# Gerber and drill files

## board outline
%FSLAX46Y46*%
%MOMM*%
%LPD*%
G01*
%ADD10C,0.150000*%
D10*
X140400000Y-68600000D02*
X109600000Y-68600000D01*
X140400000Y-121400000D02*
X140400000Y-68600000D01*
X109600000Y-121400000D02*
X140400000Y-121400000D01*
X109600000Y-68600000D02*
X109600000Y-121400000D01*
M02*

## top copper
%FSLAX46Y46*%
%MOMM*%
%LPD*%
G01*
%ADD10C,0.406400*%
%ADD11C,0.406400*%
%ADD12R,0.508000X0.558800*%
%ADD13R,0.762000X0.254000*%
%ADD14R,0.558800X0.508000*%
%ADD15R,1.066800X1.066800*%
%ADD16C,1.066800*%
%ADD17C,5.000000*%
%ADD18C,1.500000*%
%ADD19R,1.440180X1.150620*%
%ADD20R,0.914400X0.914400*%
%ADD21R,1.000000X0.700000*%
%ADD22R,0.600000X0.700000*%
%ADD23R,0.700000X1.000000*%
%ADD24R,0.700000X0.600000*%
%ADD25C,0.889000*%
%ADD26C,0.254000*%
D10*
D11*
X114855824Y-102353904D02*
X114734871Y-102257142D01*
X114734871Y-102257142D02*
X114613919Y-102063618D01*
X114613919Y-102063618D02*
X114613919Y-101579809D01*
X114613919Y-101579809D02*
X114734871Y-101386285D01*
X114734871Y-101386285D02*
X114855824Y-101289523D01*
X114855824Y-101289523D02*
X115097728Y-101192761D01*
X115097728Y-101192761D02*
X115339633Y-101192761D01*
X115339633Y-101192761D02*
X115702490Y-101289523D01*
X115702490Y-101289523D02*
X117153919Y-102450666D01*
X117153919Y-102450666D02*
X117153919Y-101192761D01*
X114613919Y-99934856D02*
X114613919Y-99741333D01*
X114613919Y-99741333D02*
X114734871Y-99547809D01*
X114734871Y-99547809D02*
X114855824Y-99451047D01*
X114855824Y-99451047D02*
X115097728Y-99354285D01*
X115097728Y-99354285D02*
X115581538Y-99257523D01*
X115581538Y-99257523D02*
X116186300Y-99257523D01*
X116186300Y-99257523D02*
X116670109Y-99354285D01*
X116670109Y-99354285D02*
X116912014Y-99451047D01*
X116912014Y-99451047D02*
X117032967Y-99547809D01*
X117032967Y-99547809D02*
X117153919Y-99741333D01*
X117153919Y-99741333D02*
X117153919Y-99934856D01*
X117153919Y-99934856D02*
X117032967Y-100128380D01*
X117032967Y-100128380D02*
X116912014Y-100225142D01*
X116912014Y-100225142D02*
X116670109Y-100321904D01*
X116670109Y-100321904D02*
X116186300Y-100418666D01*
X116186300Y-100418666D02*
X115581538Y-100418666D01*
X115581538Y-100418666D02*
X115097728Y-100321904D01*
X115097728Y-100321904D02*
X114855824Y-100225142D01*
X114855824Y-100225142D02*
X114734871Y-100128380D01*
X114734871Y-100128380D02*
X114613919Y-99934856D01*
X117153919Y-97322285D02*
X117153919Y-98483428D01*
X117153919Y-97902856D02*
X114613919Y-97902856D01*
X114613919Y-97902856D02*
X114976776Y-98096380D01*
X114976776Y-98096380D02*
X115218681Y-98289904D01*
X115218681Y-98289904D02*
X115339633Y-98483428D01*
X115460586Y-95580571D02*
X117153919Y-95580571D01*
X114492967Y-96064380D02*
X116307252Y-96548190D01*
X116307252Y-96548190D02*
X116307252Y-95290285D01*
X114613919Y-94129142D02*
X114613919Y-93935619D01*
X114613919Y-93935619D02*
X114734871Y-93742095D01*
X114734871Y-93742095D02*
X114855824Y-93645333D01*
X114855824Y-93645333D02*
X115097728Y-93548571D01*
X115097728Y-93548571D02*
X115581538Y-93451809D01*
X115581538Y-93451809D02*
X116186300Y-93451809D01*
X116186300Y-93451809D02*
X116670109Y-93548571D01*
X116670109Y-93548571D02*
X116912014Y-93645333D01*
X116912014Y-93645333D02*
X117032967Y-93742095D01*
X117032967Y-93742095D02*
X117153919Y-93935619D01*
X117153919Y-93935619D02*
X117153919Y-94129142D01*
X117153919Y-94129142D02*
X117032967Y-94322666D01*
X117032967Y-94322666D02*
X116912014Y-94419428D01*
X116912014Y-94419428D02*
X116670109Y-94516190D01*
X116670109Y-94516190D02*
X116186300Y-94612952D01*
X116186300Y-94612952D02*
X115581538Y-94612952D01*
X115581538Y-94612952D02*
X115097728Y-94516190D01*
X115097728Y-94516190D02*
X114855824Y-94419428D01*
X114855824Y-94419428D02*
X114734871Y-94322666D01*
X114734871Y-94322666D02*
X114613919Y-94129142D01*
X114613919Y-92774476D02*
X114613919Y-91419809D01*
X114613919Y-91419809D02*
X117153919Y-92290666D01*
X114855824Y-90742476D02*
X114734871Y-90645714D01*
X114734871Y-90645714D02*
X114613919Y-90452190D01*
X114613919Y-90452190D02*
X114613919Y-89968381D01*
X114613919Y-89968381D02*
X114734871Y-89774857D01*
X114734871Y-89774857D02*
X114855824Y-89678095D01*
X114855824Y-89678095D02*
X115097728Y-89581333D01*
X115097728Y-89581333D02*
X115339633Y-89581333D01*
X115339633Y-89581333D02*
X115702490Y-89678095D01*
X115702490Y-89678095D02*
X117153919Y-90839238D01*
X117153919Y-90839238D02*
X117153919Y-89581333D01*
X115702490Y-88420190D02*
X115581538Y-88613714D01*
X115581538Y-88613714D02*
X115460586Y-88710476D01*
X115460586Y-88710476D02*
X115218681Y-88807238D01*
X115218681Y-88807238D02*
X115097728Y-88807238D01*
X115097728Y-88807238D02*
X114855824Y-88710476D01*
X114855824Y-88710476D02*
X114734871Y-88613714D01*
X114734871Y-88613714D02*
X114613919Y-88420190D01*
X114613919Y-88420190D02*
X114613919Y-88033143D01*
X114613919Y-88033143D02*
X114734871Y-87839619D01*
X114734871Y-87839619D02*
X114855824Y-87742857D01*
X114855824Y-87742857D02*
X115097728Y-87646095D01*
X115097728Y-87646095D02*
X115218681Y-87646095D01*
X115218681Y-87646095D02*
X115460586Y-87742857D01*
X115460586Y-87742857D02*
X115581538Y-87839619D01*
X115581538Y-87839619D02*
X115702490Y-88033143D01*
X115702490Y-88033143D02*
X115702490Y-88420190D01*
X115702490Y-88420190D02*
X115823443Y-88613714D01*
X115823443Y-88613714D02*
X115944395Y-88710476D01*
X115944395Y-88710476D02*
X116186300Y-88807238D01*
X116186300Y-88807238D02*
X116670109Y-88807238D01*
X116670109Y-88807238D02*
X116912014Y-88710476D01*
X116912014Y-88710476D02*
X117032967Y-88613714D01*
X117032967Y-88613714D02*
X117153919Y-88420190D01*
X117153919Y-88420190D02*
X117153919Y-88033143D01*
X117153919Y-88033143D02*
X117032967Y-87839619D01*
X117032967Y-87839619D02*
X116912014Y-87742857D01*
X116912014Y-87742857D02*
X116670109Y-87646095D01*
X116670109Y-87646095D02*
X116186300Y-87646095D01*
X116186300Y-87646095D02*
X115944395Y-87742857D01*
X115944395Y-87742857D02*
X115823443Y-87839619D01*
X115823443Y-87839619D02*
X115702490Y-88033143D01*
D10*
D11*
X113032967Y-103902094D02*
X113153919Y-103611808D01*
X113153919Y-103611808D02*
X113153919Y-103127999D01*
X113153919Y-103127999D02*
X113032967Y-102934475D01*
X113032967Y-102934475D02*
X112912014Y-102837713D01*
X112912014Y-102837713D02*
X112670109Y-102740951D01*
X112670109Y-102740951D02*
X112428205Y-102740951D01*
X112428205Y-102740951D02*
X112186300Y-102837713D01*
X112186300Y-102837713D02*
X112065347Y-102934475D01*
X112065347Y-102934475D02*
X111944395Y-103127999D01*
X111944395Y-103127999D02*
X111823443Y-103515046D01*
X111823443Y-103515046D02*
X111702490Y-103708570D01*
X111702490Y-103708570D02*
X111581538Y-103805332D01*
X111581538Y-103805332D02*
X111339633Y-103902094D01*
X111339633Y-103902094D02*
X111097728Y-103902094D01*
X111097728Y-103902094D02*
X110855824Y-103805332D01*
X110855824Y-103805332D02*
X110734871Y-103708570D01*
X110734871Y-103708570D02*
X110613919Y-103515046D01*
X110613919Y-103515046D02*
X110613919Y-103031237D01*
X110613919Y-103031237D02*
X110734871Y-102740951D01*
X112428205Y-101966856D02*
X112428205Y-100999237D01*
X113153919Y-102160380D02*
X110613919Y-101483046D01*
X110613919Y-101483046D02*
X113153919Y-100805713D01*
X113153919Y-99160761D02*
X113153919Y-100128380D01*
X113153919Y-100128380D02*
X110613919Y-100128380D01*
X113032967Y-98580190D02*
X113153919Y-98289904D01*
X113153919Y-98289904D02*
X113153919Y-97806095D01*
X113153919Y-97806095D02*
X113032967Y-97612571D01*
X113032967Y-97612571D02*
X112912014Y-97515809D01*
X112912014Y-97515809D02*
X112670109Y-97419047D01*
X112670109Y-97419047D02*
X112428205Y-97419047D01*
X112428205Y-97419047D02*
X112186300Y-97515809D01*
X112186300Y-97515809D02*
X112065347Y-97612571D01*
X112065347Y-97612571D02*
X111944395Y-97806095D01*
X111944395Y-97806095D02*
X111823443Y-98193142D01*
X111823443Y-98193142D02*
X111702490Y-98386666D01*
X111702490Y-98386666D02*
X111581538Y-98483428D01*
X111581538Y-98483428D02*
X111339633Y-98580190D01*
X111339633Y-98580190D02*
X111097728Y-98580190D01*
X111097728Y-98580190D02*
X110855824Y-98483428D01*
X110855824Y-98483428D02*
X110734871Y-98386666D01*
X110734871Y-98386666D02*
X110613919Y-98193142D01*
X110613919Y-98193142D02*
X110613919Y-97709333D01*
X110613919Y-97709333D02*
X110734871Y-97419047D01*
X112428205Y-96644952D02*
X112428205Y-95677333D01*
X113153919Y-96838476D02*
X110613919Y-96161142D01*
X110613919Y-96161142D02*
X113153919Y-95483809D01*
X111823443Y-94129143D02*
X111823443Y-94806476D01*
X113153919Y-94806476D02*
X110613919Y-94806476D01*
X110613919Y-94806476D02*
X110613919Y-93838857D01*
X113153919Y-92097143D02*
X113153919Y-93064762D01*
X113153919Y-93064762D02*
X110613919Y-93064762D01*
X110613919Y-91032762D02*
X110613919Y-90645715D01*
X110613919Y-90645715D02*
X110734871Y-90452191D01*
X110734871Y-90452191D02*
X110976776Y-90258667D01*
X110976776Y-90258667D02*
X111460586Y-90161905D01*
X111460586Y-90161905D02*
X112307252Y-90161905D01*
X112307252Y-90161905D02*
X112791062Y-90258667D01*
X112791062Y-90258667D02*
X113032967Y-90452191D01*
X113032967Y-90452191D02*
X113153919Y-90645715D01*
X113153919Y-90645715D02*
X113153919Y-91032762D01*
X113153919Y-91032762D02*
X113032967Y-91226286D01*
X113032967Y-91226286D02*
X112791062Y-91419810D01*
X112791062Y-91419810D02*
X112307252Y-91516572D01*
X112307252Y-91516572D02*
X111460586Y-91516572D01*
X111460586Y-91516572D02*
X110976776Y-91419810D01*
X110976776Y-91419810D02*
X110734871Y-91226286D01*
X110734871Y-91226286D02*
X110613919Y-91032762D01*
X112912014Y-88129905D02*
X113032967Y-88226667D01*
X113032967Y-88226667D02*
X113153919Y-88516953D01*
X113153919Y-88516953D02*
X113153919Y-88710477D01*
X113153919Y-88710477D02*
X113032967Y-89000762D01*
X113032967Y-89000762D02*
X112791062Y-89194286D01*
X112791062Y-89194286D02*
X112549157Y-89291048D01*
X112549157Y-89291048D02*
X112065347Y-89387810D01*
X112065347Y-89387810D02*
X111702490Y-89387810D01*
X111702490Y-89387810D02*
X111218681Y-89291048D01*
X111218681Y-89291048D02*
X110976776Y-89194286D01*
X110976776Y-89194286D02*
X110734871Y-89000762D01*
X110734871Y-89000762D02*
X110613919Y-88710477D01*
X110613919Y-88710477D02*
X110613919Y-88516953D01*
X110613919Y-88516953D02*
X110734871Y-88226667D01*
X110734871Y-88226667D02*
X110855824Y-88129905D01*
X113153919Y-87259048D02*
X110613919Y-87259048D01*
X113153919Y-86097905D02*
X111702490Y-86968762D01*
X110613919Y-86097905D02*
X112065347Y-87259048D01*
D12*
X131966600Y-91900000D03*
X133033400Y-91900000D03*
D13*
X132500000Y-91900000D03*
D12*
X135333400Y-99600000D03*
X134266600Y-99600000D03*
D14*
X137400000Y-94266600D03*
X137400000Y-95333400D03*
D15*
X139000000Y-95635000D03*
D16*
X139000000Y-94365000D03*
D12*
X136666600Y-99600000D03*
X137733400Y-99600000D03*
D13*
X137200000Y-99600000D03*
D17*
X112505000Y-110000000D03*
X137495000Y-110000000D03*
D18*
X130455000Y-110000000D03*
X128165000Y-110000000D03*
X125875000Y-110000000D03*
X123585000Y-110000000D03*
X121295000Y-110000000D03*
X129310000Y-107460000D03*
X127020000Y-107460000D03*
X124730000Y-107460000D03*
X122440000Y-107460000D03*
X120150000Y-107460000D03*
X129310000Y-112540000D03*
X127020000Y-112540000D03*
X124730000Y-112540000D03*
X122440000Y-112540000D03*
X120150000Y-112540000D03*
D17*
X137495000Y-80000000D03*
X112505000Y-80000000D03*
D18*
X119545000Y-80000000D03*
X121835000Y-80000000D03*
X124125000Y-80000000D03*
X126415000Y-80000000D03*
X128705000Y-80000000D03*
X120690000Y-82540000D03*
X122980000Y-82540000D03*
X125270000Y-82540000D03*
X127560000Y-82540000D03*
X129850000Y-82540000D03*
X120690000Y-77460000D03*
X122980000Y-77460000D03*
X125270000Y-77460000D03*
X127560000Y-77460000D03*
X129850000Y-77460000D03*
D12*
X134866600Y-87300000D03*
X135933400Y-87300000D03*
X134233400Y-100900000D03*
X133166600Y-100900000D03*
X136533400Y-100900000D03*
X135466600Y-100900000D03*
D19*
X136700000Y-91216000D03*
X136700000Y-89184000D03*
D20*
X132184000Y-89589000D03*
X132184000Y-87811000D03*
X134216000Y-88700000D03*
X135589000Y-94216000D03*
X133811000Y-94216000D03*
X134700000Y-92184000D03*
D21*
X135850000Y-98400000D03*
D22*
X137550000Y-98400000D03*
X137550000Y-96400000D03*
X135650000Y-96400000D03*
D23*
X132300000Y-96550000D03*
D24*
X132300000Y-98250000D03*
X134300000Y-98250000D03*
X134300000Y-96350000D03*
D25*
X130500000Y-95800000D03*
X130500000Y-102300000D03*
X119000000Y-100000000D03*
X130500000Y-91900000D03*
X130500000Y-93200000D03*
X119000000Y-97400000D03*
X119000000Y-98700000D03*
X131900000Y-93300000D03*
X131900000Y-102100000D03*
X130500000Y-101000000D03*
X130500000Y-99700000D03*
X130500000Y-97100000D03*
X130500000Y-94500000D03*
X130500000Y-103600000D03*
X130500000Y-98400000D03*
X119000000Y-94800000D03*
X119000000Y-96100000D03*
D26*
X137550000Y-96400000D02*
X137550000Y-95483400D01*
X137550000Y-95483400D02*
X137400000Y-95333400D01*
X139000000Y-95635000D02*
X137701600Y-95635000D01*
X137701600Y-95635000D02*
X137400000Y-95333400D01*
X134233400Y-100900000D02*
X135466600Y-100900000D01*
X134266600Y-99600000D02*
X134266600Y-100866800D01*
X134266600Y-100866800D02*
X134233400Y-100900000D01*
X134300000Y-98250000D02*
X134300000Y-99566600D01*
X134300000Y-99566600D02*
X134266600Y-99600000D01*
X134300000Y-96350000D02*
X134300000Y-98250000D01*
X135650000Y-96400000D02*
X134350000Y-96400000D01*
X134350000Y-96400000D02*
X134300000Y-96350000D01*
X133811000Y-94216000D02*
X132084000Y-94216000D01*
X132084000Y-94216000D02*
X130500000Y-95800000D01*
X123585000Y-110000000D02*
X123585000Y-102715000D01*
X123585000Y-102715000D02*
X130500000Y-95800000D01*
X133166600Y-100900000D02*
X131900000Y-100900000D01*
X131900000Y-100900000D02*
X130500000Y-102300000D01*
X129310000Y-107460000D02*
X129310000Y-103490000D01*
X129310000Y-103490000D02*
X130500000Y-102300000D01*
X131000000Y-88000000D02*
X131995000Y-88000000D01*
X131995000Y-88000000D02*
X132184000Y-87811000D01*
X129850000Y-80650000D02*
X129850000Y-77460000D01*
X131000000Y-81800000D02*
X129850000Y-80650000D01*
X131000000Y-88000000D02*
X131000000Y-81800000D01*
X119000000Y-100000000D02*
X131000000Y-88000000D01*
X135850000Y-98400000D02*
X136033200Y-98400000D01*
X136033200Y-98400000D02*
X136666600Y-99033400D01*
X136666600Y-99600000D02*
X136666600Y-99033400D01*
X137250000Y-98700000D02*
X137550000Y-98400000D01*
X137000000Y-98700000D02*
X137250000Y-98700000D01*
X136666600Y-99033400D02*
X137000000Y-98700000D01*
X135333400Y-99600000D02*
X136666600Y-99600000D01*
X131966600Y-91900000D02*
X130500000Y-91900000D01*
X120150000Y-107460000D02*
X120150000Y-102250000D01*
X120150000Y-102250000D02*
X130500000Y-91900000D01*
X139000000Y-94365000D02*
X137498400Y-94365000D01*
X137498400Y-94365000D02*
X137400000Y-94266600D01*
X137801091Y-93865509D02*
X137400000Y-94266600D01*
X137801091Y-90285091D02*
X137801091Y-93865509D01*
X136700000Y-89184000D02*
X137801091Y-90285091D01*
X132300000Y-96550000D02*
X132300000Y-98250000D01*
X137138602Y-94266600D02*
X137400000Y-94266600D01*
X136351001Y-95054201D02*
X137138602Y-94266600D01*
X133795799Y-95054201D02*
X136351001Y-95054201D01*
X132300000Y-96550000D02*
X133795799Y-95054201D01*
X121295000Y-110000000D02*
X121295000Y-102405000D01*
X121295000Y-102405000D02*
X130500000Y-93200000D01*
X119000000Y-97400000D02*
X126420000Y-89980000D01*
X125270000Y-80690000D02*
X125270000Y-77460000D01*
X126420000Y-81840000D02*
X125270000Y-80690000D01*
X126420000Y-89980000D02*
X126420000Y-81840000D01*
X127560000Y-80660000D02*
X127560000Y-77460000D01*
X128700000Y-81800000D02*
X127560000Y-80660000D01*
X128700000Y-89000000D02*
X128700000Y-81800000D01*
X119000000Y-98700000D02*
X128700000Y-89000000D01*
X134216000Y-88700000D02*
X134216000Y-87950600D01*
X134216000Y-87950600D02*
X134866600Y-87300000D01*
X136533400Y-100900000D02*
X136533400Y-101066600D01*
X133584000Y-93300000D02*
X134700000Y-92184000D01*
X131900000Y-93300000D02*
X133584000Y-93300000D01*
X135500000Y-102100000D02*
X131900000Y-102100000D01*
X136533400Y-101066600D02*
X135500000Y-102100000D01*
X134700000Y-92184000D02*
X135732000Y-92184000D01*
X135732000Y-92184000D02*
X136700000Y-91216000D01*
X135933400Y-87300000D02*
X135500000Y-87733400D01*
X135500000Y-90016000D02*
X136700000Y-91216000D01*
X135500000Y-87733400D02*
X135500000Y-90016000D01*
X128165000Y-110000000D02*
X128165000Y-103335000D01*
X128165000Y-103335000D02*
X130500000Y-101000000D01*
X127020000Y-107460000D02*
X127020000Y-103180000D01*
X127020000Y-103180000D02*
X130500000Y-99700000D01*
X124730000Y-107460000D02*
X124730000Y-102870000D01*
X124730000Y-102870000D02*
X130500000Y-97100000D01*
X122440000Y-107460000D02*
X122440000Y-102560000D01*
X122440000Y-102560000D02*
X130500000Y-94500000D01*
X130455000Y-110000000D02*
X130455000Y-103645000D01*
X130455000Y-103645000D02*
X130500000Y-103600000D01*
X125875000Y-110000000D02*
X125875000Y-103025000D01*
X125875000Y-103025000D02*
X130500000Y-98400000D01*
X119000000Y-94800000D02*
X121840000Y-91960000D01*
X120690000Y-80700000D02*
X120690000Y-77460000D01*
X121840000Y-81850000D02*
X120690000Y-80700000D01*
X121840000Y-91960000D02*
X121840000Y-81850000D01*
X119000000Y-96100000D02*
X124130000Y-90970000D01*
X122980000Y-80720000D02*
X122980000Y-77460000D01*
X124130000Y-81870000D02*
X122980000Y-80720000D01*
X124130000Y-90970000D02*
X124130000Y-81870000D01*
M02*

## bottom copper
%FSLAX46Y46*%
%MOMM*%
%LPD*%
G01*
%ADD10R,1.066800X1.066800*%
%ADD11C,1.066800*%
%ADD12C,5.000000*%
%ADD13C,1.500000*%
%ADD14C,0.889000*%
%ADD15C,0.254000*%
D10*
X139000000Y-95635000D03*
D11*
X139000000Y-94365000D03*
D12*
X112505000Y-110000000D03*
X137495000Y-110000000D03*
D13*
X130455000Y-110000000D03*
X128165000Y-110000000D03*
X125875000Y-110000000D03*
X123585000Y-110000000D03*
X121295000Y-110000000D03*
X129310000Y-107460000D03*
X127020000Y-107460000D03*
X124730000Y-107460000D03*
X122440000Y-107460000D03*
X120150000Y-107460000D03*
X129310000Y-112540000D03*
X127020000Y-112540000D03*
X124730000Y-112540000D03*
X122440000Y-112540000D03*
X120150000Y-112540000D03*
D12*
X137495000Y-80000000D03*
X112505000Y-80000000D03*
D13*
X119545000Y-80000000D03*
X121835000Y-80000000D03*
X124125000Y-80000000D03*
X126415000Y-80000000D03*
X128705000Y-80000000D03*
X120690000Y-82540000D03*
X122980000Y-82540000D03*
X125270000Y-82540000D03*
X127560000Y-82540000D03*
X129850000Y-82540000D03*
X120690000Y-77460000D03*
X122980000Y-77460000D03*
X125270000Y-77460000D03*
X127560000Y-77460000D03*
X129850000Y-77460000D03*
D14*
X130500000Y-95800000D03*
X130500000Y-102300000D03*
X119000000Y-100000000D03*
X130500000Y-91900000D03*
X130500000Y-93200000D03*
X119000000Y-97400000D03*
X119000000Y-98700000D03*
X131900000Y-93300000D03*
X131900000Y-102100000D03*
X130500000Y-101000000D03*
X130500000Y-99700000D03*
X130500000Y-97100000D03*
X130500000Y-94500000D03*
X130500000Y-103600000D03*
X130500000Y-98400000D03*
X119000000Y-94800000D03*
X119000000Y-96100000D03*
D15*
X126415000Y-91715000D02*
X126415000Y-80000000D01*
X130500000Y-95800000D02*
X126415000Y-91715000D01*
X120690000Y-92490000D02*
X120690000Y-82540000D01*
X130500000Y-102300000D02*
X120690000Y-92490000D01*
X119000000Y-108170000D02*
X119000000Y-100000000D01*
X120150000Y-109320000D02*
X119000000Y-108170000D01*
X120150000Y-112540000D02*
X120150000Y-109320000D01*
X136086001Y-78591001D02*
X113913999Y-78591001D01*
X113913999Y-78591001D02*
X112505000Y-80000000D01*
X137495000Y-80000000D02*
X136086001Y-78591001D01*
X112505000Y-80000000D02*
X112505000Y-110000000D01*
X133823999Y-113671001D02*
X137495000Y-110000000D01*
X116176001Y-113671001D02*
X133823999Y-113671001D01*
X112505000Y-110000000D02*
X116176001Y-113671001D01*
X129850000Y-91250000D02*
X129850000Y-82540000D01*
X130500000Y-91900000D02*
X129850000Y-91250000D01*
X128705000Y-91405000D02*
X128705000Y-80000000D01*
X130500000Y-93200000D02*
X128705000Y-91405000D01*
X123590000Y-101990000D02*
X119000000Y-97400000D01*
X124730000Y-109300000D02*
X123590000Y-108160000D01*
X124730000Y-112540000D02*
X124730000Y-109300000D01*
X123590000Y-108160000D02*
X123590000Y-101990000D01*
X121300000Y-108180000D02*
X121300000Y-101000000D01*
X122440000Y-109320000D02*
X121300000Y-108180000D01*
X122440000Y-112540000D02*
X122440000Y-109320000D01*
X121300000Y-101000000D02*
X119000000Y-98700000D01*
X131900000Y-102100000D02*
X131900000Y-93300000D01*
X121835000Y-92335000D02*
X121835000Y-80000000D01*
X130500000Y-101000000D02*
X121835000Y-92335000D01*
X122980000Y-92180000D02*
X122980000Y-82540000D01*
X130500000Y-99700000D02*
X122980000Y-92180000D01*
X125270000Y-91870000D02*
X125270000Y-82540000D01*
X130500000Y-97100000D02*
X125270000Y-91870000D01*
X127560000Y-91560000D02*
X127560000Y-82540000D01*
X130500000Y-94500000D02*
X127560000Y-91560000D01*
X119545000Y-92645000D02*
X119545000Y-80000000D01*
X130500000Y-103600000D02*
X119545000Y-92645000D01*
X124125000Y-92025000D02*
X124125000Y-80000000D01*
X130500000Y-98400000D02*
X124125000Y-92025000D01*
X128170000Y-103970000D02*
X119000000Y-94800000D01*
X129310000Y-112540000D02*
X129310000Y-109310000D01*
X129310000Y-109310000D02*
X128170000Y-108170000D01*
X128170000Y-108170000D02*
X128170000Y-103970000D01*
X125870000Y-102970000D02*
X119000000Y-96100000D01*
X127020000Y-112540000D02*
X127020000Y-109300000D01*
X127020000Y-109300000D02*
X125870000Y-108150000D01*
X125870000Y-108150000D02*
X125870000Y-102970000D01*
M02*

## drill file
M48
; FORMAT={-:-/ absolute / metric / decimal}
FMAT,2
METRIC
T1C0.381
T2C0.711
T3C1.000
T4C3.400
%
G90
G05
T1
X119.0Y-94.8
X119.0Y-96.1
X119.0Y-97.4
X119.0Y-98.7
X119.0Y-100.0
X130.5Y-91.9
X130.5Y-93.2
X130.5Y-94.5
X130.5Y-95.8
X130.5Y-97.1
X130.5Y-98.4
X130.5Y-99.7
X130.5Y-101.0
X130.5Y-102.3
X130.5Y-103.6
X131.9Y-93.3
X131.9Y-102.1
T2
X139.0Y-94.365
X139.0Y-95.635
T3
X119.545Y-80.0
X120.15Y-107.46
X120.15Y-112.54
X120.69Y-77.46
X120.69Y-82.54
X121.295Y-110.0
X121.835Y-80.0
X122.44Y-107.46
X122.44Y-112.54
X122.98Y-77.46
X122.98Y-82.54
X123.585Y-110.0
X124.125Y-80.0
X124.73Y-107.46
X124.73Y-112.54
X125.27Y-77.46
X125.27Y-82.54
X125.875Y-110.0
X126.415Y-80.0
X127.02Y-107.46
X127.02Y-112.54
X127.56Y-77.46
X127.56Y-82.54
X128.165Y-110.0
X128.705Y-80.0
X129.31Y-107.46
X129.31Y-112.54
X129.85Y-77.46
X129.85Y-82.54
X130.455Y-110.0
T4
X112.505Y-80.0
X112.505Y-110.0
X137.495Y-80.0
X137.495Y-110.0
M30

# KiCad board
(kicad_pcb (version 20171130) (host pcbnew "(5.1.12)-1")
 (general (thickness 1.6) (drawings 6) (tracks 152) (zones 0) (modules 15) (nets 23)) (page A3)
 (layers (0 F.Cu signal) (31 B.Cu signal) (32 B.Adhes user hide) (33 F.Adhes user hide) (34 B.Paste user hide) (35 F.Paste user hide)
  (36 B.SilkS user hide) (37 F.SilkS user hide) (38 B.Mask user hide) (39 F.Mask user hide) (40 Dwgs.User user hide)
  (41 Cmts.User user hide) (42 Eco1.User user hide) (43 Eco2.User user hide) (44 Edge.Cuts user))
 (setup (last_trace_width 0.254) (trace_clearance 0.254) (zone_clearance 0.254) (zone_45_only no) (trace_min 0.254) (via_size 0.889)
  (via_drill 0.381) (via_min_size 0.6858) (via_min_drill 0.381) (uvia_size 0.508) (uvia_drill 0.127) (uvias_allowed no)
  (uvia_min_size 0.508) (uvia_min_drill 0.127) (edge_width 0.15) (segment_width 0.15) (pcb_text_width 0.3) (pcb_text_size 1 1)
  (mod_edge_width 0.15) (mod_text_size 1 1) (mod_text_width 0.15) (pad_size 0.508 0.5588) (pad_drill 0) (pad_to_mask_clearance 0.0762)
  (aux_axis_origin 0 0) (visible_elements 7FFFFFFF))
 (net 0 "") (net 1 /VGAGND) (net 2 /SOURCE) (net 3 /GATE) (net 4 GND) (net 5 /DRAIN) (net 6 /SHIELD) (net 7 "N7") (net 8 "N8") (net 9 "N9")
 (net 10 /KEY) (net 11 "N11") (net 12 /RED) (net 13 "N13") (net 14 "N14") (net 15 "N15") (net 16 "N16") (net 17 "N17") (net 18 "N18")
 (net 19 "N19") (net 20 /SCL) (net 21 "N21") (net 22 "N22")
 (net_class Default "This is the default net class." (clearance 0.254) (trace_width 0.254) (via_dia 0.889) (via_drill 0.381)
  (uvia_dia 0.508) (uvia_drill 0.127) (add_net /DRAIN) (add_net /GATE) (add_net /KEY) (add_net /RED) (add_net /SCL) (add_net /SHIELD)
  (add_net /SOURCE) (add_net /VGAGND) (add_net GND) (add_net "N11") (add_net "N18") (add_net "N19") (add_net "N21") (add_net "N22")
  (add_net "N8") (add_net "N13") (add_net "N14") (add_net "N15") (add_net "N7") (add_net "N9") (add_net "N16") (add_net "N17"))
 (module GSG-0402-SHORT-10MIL (layer F.Cu) (at 132.5 91.9 180) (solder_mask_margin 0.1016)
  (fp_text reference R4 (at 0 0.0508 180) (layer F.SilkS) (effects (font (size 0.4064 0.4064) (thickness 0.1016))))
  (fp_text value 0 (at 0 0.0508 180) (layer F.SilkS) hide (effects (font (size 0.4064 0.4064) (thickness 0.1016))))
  (pad 2 smd rect (at 0.5334 0 180) (size 0.508 0.5588) (layers F.Cu F.Mask) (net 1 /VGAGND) (solder_mask_margin 0.1016))
  (pad 1 smd rect (at -0.5334 0 180) (size 0.508 0.5588) (layers F.Cu F.Mask) (die_length -1518.485687) (solder_mask_margin 0.1016))
  (pad "" smd rect (at 0 0 180) (size 0.762 0.254) (layers F.Cu F.Mask)))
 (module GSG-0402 (layer F.Cu) (at 134.8 99.6) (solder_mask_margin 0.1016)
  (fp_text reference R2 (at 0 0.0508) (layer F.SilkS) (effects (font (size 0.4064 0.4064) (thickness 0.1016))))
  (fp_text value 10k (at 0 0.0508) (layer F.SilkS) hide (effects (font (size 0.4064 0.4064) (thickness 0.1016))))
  (pad 2 smd rect (at 0.5334 0) (size 0.508 0.5588) (layers F.Cu F.Paste F.Mask) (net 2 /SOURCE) (solder_mask_margin 0.1016))
  (pad 1 smd rect (at -0.5334 0) (size 0.508 0.5588) (layers F.Cu F.Paste F.Mask) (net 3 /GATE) (die_length -1518.485687)
   (solder_mask_margin 0.1016)))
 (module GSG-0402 (layer F.Cu) (at 137.4 94.8 90) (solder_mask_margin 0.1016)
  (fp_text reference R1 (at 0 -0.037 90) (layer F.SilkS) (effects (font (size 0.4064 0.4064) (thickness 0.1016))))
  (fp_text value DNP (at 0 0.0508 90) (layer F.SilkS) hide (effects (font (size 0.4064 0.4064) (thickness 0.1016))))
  (pad 2 smd rect (at 0.5334 0 90) (size 0.508 0.5588) (layers F.Cu F.Paste F.Mask) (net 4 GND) (solder_mask_margin 0.1016))
  (pad 1 smd rect (at -0.5334 0 90) (size 0.508 0.5588) (layers F.Cu F.Paste F.Mask) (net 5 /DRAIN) (die_length -1518.485687)
   (solder_mask_margin 0.1016)))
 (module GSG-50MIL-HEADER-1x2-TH (layer F.Cu) (at 139 95 90)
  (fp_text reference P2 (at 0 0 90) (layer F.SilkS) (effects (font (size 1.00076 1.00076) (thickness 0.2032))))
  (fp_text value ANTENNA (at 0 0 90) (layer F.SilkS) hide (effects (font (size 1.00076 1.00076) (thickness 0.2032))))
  (pad 1 thru_hole rect (at -0.635 0 90) (size 1.0668 1.0668) (drill 0.7112) (layers *.Cu *.Mask) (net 5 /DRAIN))
  (pad 2 thru_hole circle (at 0.635 0 90) (size 1.0668 1.0668) (drill 0.7112) (layers *.Cu *.Mask) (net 4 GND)))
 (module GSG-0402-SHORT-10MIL (layer F.Cu) (at 137.2 99.6 180) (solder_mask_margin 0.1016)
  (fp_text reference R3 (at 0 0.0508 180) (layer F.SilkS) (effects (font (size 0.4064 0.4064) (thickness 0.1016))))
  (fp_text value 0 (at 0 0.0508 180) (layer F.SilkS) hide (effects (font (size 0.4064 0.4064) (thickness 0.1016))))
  (pad 2 smd rect (at 0.5334 0 180) (size 0.508 0.5588) (layers F.Cu F.Mask) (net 2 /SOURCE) (solder_mask_margin 0.1016))
  (pad 1 smd rect (at -0.5334 0 180) (size 0.508 0.5588) (layers F.Cu F.Mask) (die_length -1518.485687) (solder_mask_margin 0.1016))
  (pad "" smd rect (at 0 0 180) (size 0.762 0.254) (layers F.Cu F.Mask)))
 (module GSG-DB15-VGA (layer F.Cu) (at 125 110)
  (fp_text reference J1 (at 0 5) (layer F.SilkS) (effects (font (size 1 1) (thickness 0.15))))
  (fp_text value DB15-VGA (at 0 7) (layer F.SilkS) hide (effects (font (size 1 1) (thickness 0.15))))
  (pad 0 thru_hole circle (at -12.495 0) (size 5 5) (drill 3.4) (layers *.Cu *.Mask) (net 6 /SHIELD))
  (pad 0 thru_hole circle (at 12.495 0) (size 5 5) (drill 3.4) (layers *.Cu *.Mask) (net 6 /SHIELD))
  (pad 6 thru_hole circle (at 5.455 0) (size 1.5 1.5) (drill 1) (layers *.Cu *.Mask) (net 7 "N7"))
  (pad 7 thru_hole circle (at 3.165 0) (size 1.5 1.5) (drill 1) (layers *.Cu *.Mask) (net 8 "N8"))
  (pad 8 thru_hole circle (at 0.875 0) (size 1.5 1.5) (drill 1) (layers *.Cu *.Mask) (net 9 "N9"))
  (pad 9 thru_hole circle (at -1.415 0) (size 1.5 1.5) (drill 1) (layers *.Cu *.Mask) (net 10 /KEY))
  (pad 10 thru_hole circle (at -3.705 0) (size 1.5 1.5) (drill 1) (layers *.Cu *.Mask) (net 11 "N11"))
  (pad 1 thru_hole circle (at 4.31 -2.54) (size 1.5 1.5) (drill 1) (layers *.Cu *.Mask) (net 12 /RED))
  (pad 2 thru_hole circle (at 2.02 -2.54) (size 1.5 1.5) (drill 1) (layers *.Cu *.Mask) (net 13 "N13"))
  (pad 3 thru_hole circle (at -0.27 -2.54) (size 1.5 1.5) (drill 1) (layers *.Cu *.Mask) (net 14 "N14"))
  (pad 4 thru_hole circle (at -2.56 -2.54) (size 1.5 1.5) (drill 1) (layers *.Cu *.Mask) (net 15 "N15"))
  (pad 5 thru_hole circle (at -4.85 -2.54) (size 1.5 1.5) (drill 1) (layers *.Cu *.Mask) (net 1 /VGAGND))
  (pad 11 thru_hole circle (at 4.31 2.54) (size 1.5 1.5) (drill 1) (layers *.Cu *.Mask) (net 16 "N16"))
  (pad 12 thru_hole circle (at 2.02 2.54) (size 1.5 1.5) (drill 1) (layers *.Cu *.Mask) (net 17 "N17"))
  (pad 13 thru_hole circle (at -0.27 2.54) (size 1.5 1.5) (drill 1) (layers *.Cu *.Mask) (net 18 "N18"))
  (pad 14 thru_hole circle (at -2.56 2.54) (size 1.5 1.5) (drill 1) (layers *.Cu *.Mask) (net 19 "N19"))
  (pad 15 thru_hole circle (at -4.85 2.54) (size 1.5 1.5) (drill 1) (layers *.Cu *.Mask) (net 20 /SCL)))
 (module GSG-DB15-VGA (layer F.Cu) (at 125 80 180)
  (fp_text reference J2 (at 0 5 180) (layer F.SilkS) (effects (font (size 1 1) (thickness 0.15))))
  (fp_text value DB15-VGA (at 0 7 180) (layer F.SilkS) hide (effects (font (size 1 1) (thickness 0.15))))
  (pad 0 thru_hole circle (at -12.495 0 180) (size 5 5) (drill 3.4) (layers *.Cu *.Mask) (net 6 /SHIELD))
  (pad 0 thru_hole circle (at 12.495 0 180) (size 5 5) (drill 3.4) (layers *.Cu *.Mask) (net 6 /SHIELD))
  (pad 6 thru_hole circle (at 5.455 0 180) (size 1.5 1.5) (drill 1) (layers *.Cu *.Mask) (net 7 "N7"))
  (pad 7 thru_hole circle (at 3.165 0 180) (size 1.5 1.5) (drill 1) (layers *.Cu *.Mask) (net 8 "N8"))
  (pad 8 thru_hole circle (at 0.875 0 180) (size 1.5 1.5) (drill 1) (layers *.Cu *.Mask) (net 9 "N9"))
  (pad 9 thru_hole circle (at -1.415 0 180) (size 1.5 1.5) (drill 1) (layers *.Cu *.Mask) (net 10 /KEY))
  (pad 10 thru_hole circle (at -3.705 0 180) (size 1.5 1.5) (drill 1) (layers *.Cu *.Mask) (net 11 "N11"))
  (pad 1 thru_hole circle (at 4.31 -2.54 180) (size 1.5 1.5) (drill 1) (layers *.Cu *.Mask) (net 12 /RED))
  (pad 2 thru_hole circle (at 2.02 -2.54 180) (size 1.5 1.5) (drill 1) (layers *.Cu *.Mask) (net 13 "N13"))
  (pad 3 thru_hole circle (at -0.27 -2.54 180) (size 1.5 1.5) (drill 1) (layers *.Cu *.Mask) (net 14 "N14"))
  (pad 4 thru_hole circle (at -2.56 -2.54 180) (size 1.5 1.5) (drill 1) (layers *.Cu *.Mask) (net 15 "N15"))
  (pad 5 thru_hole circle (at -4.85 -2.54 180) (size 1.5 1.5) (drill 1) (layers *.Cu *.Mask) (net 1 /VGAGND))
  (pad 11 thru_hole circle (at 4.31 2.54 180) (size 1.5 1.5) (drill 1) (layers *.Cu *.Mask) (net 16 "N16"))
  (pad 12 thru_hole circle (at 2.02 2.54 180) (size 1.5 1.5) (drill 1) (layers *.Cu *.Mask) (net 17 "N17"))
  (pad 13 thru_hole circle (at -0.27 2.54 180) (size 1.5 1.5) (drill 1) (layers *.Cu *.Mask) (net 18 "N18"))
  (pad 14 thru_hole circle (at -2.56 2.54 180) (size 1.5 1.5) (drill 1) (layers *.Cu *.Mask) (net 19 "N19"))
  (pad 15 thru_hole circle (at -4.85 2.54 180) (size 1.5 1.5) (drill 1) (layers *.Cu *.Mask) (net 20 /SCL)))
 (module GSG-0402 (layer F.Cu) (at 135.4 87.3 180) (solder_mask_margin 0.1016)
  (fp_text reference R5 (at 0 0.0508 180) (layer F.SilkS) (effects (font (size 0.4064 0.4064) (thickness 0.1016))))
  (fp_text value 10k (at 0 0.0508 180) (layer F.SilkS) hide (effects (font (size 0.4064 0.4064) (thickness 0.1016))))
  (pad 2 smd rect (at 0.5334 0 180) (size 0.508 0.5588) (layers F.Cu F.Paste F.Mask) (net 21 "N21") (solder_mask_margin 0.1016))
  (pad 1 smd rect (at -0.5334 0 180) (size 0.508 0.5588) (layers F.Cu F.Paste F.Mask) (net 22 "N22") (die_length -1518.485687)
   (solder_mask_margin 0.1016)))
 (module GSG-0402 (layer F.Cu) (at 133.7 100.9) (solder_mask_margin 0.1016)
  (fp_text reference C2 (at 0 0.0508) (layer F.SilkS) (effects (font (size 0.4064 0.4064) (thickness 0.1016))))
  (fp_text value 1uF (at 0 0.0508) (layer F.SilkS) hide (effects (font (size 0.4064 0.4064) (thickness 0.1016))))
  (pad 2 smd rect (at 0.5334 0) (size 0.508 0.5588) (layers F.Cu F.Paste F.Mask) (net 3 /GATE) (solder_mask_margin 0.1016))
  (pad 1 smd rect (at -0.5334 0) (size 0.508 0.5588) (layers F.Cu F.Paste F.Mask) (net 12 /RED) (die_length -1518.485687)
   (solder_mask_margin 0.1016)))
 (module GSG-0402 (layer F.Cu) (at 136 100.9) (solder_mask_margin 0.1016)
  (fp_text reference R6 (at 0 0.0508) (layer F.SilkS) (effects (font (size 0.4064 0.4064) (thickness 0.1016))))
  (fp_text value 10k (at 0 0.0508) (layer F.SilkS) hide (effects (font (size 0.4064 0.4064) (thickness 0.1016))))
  (pad 2 smd rect (at 0.5334 0) (size 0.508 0.5588) (layers F.Cu F.Paste F.Mask) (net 22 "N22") (solder_mask_margin 0.1016))
  (pad 1 smd rect (at -0.5334 0) (size 0.508 0.5588) (layers F.Cu F.Paste F.Mask) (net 3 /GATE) (die_length -1518.485687)
   (solder_mask_margin 0.1016)))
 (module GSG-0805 (layer F.Cu) (at 136.7 90.2 270) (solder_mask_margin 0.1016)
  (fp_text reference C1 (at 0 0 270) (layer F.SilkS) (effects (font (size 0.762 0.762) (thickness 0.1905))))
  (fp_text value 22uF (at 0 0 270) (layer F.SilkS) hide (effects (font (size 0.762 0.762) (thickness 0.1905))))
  (pad 2 smd rect (at 1.016 0 270) (size 1.15062 1.44018) (layers F.Cu F.Paste F.Mask) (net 22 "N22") (die_length 0.08128)
   (solder_mask_margin 0.1016) (clearance 0.1778))
  (pad 1 smd rect (at -1.016 0 270) (size 1.15062 1.44018) (layers F.Cu F.Paste F.Mask) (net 4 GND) (die_length -1518.485687)
   (solder_mask_margin 0.1016) (clearance 0.1778)))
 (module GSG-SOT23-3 (layer F.Cu) (at 133.2 88.7 90)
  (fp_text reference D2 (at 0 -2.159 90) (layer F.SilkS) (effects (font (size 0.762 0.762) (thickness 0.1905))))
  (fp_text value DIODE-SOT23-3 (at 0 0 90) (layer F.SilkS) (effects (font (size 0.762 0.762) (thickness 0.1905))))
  (pad 2 smd rect (at -0.889 -1.016 90) (size 0.9144 0.9144) (layers F.Cu F.Paste F.Mask) (die_length 0.00762))
  (pad 1 smd rect (at 0.889 -1.016 90) (size 0.9144 0.9144) (layers F.Cu F.Paste F.Mask) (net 20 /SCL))
  (pad 3 smd rect (at 0 1.016 90) (size 0.9144 0.9144) (layers F.Cu F.Paste F.Mask) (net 21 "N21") (die_length 0.28194)))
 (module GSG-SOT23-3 (layer F.Cu) (at 134.7 93.2 180)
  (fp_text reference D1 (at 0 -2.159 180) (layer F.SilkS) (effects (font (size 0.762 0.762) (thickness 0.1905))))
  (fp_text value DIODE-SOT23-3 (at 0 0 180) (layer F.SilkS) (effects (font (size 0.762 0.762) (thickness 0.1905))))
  (pad 2 smd rect (at -0.889 -1.016 180) (size 0.9144 0.9144) (layers F.Cu F.Paste F.Mask) (die_length 0.00762))
  (pad 1 smd rect (at 0.889 -1.016 180) (size 0.9144 0.9144) (layers F.Cu F.Paste F.Mask) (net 10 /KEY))
  (pad 3 smd rect (at 0 1.016 180) (size 0.9144 0.9144) (layers F.Cu F.Paste F.Mask) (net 22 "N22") (die_length 0.28194)))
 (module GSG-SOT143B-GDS (layer F.Cu) (at 136.6 97.4)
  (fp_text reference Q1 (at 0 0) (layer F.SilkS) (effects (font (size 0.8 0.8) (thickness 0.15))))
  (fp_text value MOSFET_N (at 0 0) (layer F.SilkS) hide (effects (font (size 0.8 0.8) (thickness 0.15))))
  (pad B smd rect (at -0.75 1) (size 1 0.7) (layers F.Cu F.Paste F.Mask) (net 2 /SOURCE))
  (pad S smd rect (at 0.95 1) (size 0.6 0.7) (layers F.Cu F.Paste F.Mask) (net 2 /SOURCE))
  (pad D smd rect (at 0.95 -1) (size 0.6 0.7) (layers F.Cu F.Paste F.Mask) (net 5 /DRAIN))
  (pad G smd rect (at -0.95 -1) (size 0.6 0.7) (layers F.Cu F.Paste F.Mask) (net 3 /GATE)))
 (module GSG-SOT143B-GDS (layer F.Cu) (at 133.3 97.3 270)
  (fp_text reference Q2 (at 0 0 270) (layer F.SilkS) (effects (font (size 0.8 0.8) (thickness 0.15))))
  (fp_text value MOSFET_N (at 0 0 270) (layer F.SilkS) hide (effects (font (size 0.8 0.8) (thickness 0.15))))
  (pad B smd rect (at -0.75 1 270) (size 1 0.7) (layers F.Cu F.Paste F.Mask) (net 4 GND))
  (pad S smd rect (at 0.95 1 270) (size 0.6 0.7) (layers F.Cu F.Paste F.Mask) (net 4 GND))
  (pad D smd rect (at 0.95 -1 270) (size 0.6 0.7) (layers F.Cu F.Paste F.Mask) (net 3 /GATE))
  (pad G smd rect (at -0.95 -1 270) (size 0.6 0.7) (layers F.Cu F.Paste F.Mask) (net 3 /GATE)))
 (gr_line (start 140.4 68.6) (end 109.6 68.6) (angle 90) (layer Edge.Cuts) (width 0.15))
 (gr_line (start 140.4 121.4) (end 140.4 68.6) (angle 90) (layer Edge.Cuts) (width 0.15))
 (gr_line (start 109.6 121.4) (end 140.4 121.4) (angle 90) (layer Edge.Cuts) (width 0.15))
 (gr_line (start 109.6 68.6) (end 109.6 121.4) (angle 90) (layer Edge.Cuts) (width 0.15))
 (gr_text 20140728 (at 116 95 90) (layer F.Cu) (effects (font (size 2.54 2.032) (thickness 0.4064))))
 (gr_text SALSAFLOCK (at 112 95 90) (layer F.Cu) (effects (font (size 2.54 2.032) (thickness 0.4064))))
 (segment (start 137.55 96.4) (end 137.55 95.4834) (width 0.254) (layer F.Cu) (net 5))
 (segment (start 137.55 95.4834) (end 137.4 95.3334) (width 0.254) (layer F.Cu) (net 5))
 (segment (start 139 95.635) (end 137.7016 95.635) (width 0.254) (layer F.Cu) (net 5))
 (segment (start 137.7016 95.635) (end 137.4 95.3334) (width 0.254) (layer F.Cu) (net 5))
 (segment (start 134.2334 100.9) (end 135.4666 100.9) (width 0.254) (layer F.Cu) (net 3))
 (segment (start 134.2666 99.6) (end 134.2666 100.8668) (width 0.254) (layer F.Cu) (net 3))
 (segment (start 134.2666 100.8668) (end 134.2334 100.9) (width 0.254) (layer F.Cu) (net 3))
 (segment (start 134.3 98.25) (end 134.3 99.5666) (width 0.254) (layer F.Cu) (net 3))
 (segment (start 134.3 99.5666) (end 134.2666 99.6) (width 0.254) (layer F.Cu) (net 3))
 (segment (start 134.3 96.35) (end 134.3 98.25) (width 0.254) (layer F.Cu) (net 3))
 (segment (start 135.65 96.4) (end 134.35 96.4) (width 0.254) (layer F.Cu) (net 3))
 (segment (start 134.35 96.4) (end 134.3 96.35) (width 0.254) (layer F.Cu) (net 3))
 (segment (start 133.811 94.216) (end 132.084 94.216) (width 0.254) (layer F.Cu) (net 10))
 (segment (start 132.084 94.216) (end 130.5 95.8) (width 0.254) (layer F.Cu) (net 10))
 (segment (start 123.585 110) (end 123.585 102.715) (width 0.254) (layer F.Cu) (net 10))
 (segment (start 126.415 91.715) (end 126.415 80) (width 0.254) (layer B.Cu) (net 10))
 (segment (start 130.5 95.8) (end 126.415 91.715) (width 0.254) (layer B.Cu) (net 10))
 (segment (start 123.585 102.715) (end 130.5 95.8) (width 0.254) (layer F.Cu) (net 10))
 (segment (start 133.1666 100.9) (end 131.9 100.9) (width 0.254) (layer F.Cu) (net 12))
 (segment (start 131.9 100.9) (end 130.5 102.3) (width 0.254) (layer F.Cu) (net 12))
 (segment (start 129.31 107.46) (end 129.31 103.49) (width 0.254) (layer F.Cu) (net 12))
 (segment (start 120.69 92.49) (end 120.69 82.54) (width 0.254) (layer B.Cu) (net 12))
 (segment (start 130.5 102.3) (end 120.69 92.49) (width 0.254) (layer B.Cu) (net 12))
 (segment (start 129.31 103.49) (end 130.5 102.3) (width 0.254) (layer F.Cu) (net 12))
 (segment (start 131 88) (end 131.995 88) (width 0.254) (layer F.Cu) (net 20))
 (segment (start 131.995 88) (end 132.184 87.811) (width 0.254) (layer F.Cu) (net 20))
 (segment (start 119 108.17) (end 119 100) (width 0.254) (layer B.Cu) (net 20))
 (segment (start 120.15 109.32) (end 119 108.17) (width 0.254) (layer B.Cu) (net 20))
 (segment (start 120.15 112.54) (end 120.15 109.32) (width 0.254) (layer B.Cu) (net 20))
 (segment (start 129.85 80.65) (end 129.85 77.46) (width 0.254) (layer F.Cu) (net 20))
 (segment (start 131 81.8) (end 129.85 80.65) (width 0.254) (layer F.Cu) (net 20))
 (segment (start 131 88) (end 131 81.8) (width 0.254) (layer F.Cu) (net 20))
 (segment (start 119 100) (end 131 88) (width 0.254) (layer F.Cu) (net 20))
 (segment (start 136.086001 78.591001) (end 113.913999 78.591001) (width 0.254) (layer B.Cu) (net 6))
 (segment (start 113.913999 78.591001) (end 112.505 80) (width 0.254) (layer B.Cu) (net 6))
 (segment (start 137.495 80) (end 136.086001 78.591001) (width 0.254) (layer B.Cu) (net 6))
 (segment (start 112.505 80) (end 112.505 110) (width 0.254) (layer B.Cu) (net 6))
 (segment (start 133.823999 113.671001) (end 137.495 110) (width 0.254) (layer B.Cu) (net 6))
 (segment (start 116.176001 113.671001) (end 133.823999 113.671001) (width 0.254) (layer B.Cu) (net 6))
 (segment (start 112.505 110) (end 116.176001 113.671001) (width 0.254) (layer B.Cu) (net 6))
 (segment (start 135.85 98.4) (end 136.0332 98.4) (width 0.254) (layer F.Cu) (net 2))
 (segment (start 136.0332 98.4) (end 136.6666 99.0334) (width 0.254) (layer F.Cu) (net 2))
 (segment (start 136.6666 99.6) (end 136.6666 99.0334) (width 0.254) (layer F.Cu) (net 2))
 (segment (start 137.25 98.7) (end 137.55 98.4) (width 0.254) (layer F.Cu) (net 2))
 (segment (start 137 98.7) (end 137.25 98.7) (width 0.254) (layer F.Cu) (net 2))
 (segment (start 136.6666 99.0334) (end 137 98.7) (width 0.254) (layer F.Cu) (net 2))
 (segment (start 135.3334 99.6) (end 136.6666 99.6) (width 0.254) (layer F.Cu) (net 2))
 (segment (start 131.9666 91.9) (end 130.5 91.9) (width 0.254) (layer F.Cu) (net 1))
 (segment (start 120.15 107.46) (end 120.15 102.25) (width 0.254) (layer F.Cu) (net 1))
 (segment (start 129.85 91.25) (end 129.85 82.54) (width 0.254) (layer B.Cu) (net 1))
 (segment (start 130.5 91.9) (end 129.85 91.25) (width 0.254) (layer B.Cu) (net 1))
 (segment (start 120.15 102.25) (end 130.5 91.9) (width 0.254) (layer F.Cu) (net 1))
 (segment (start 139 94.365) (end 137.4984 94.365) (width 0.254) (layer F.Cu) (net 4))
 (segment (start 137.4984 94.365) (end 137.4 94.2666) (width 0.254) (layer F.Cu) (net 4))
 (segment (start 137.801091 93.865509) (end 137.4 94.2666) (width 0.254) (layer F.Cu) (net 4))
 (segment (start 137.801091 90.285091) (end 137.801091 93.865509) (width 0.254) (layer F.Cu) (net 4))
 (segment (start 136.7 89.184) (end 137.801091 90.285091) (width 0.254) (layer F.Cu) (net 4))
 (segment (start 132.3 96.55) (end 132.3 98.25) (width 0.254) (layer F.Cu) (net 4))
 (segment (start 137.138602 94.2666) (end 137.4 94.2666) (width 0.254) (layer F.Cu) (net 4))
 (segment (start 136.351001 95.054201) (end 137.138602 94.2666) (width 0.254) (layer F.Cu) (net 4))
 (segment (start 133.795799 95.054201) (end 136.351001 95.054201) (width 0.254) (layer F.Cu) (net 4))
 (segment (start 132.3 96.55) (end 133.795799 95.054201) (width 0.254) (layer F.Cu) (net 4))
 (segment (start 121.295 110) (end 121.295 102.405) (width 0.254) (layer F.Cu) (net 11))
 (segment (start 128.705 91.405) (end 128.705 80) (width 0.254) (layer B.Cu) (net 11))
 (segment (start 130.5 93.2) (end 128.705 91.405) (width 0.254) (layer B.Cu) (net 11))
 (segment (start 121.295 102.405) (end 130.5 93.2) (width 0.254) (layer F.Cu) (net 11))
 (segment (start 119 97.4) (end 126.42 89.98) (width 0.254) (layer F.Cu) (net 18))
 (segment (start 123.59 101.99) (end 119 97.4) (width 0.254) (layer B.Cu) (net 18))
 (segment (start 124.73 109.3) (end 123.59 108.16) (width 0.254) (layer B.Cu) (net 18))
 (segment (start 124.73 112.54) (end 124.73 109.3) (width 0.254) (layer B.Cu) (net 18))
 (segment (start 123.59 108.16) (end 123.59 101.99) (width 0.254) (layer B.Cu) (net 18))
 (segment (start 125.27 80.69) (end 125.27 77.46) (width 0.254) (layer F.Cu) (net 18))
 (segment (start 126.42 81.84) (end 125.27 80.69) (width 0.254) (layer F.Cu) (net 18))
 (segment (start 126.42 89.98) (end 126.42 81.84) (width 0.254) (layer F.Cu) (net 18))
 (segment (start 121.3 108.18) (end 121.3 101) (width 0.254) (layer B.Cu) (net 19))
 (segment (start 122.44 109.32) (end 121.3 108.18) (width 0.254) (layer B.Cu) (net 19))
 (segment (start 122.44 112.54) (end 122.44 109.32) (width 0.254) (layer B.Cu) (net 19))
 (segment (start 127.56 80.66) (end 127.56 77.46) (width 0.254) (layer F.Cu) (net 19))
 (segment (start 128.7 81.8) (end 127.56 80.66) (width 0.254) (layer F.Cu) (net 19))
 (segment (start 128.7 89) (end 128.7 81.8) (width 0.254) (layer F.Cu) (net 19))
 (segment (start 119 98.7) (end 128.7 89) (width 0.254) (layer F.Cu) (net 19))
 (segment (start 121.3 101) (end 119 98.7) (width 0.254) (layer B.Cu) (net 19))
 (segment (start 134.216 88.7) (end 134.216 87.9506) (width 0.254) (layer F.Cu) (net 21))
 (segment (start 134.216 87.9506) (end 134.8666 87.3) (width 0.254) (layer F.Cu) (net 21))
 (segment (start 136.5334 100.9) (end 136.5334 101.0666) (width 0.254) (layer F.Cu) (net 22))
 (segment (start 133.584 93.3) (end 134.7 92.184) (width 0.254) (layer F.Cu) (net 22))
 (segment (start 131.9 93.3) (end 133.584 93.3) (width 0.254) (layer F.Cu) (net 22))
 (segment (start 131.9 102.1) (end 131.9 93.3) (width 0.254) (layer B.Cu) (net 22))
 (segment (start 135.5 102.1) (end 131.9 102.1) (width 0.254) (layer F.Cu) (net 22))
 (segment (start 136.5334 101.0666) (end 135.5 102.1) (width 0.254) (layer F.Cu) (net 22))
 (segment (start 134.7 92.184) (end 135.732 92.184) (width 0.254) (layer F.Cu) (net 22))
 (segment (start 135.732 92.184) (end 136.7 91.216) (width 0.254) (layer F.Cu) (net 22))
 (segment (start 135.9334 87.3) (end 135.5 87.7334) (width 0.254) (layer F.Cu) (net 22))
 (segment (start 135.5 90.016) (end 136.7 91.216) (width 0.254) (layer F.Cu) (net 22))
 (segment (start 135.5 87.7334) (end 135.5 90.016) (width 0.254) (layer F.Cu) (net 22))
 (segment (start 128.165 110) (end 128.165 103.335) (width 0.254) (layer F.Cu) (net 8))
 (segment (start 121.835 92.335) (end 121.835 80) (width 0.254) (layer B.Cu) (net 8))
 (segment (start 130.5 101) (end 121.835 92.335) (width 0.254) (layer B.Cu) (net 8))
 (segment (start 128.165 103.335) (end 130.5 101) (width 0.254) (layer F.Cu) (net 8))
 (segment (start 127.02 107.46) (end 127.02 103.18) (width 0.254) (layer F.Cu) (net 13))
 (segment (start 122.98 92.18) (end 122.98 82.54) (width 0.254) (layer B.Cu) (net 13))
 (segment (start 130.5 99.7) (end 122.98 92.18) (width 0.254) (layer B.Cu) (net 13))
 (segment (start 127.02 103.18) (end 130.5 99.7) (width 0.254) (layer F.Cu) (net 13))
 (segment (start 124.73 107.46) (end 124.73 102.87) (width 0.254) (layer F.Cu) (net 14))
 (segment (start 125.27 91.87) (end 125.27 82.54) (width 0.254) (layer B.Cu) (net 14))
 (segment (start 130.5 97.1) (end 125.27 91.87) (width 0.254) (layer B.Cu) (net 14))
 (segment (start 124.73 102.87) (end 130.5 97.1) (width 0.254) (layer F.Cu) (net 14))
 (segment (start 122.44 107.46) (end 122.44 102.56) (width 0.254) (layer F.Cu) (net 15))
 (segment (start 127.56 91.56) (end 127.56 82.54) (width 0.254) (layer B.Cu) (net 15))
 (segment (start 130.5 94.5) (end 127.56 91.56) (width 0.254) (layer B.Cu) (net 15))
 (segment (start 122.44 102.56) (end 130.5 94.5) (width 0.254) (layer F.Cu) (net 15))
 (segment (start 130.455 110) (end 130.455 103.645) (width 0.254) (layer F.Cu) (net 7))
 (segment (start 119.545 92.645) (end 119.545 80) (width 0.254) (layer B.Cu) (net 7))
 (segment (start 130.5 103.6) (end 119.545 92.645) (width 0.254) (layer B.Cu) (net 7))
 (segment (start 130.455 103.645) (end 130.5 103.6) (width 0.254) (layer F.Cu) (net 7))
 (segment (start 125.875 110) (end 125.875 103.025) (width 0.254) (layer F.Cu) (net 9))
 (segment (start 124.125 92.025) (end 124.125 80) (width 0.254) (layer B.Cu) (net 9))
 (segment (start 130.5 98.4) (end 124.125 92.025) (width 0.254) (layer B.Cu) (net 9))
 (segment (start 125.875 103.025) (end 130.5 98.4) (width 0.254) (layer F.Cu) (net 9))
 (segment (start 119 94.8) (end 121.84 91.96) (width 0.254) (layer F.Cu) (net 16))
 (segment (start 128.17 103.97) (end 119 94.8) (width 0.254) (layer B.Cu) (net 16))
 (segment (start 129.31 112.54) (end 129.31 109.31) (width 0.254) (layer B.Cu) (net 16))
 (segment (start 129.31 109.31) (end 128.17 108.17) (width 0.254) (layer B.Cu) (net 16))
 (segment (start 128.17 108.17) (end 128.17 103.97) (width 0.254) (layer B.Cu) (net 16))
 (segment (start 120.69 80.7) (end 120.69 77.46) (width 0.254) (layer F.Cu) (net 16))
 (segment (start 121.84 81.85) (end 120.69 80.7) (width 0.254) (layer F.Cu) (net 16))
 (segment (start 121.84 91.96) (end 121.84 81.85) (width 0.254) (layer F.Cu) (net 16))
 (segment (start 119 96.1) (end 124.13 90.97) (width 0.254) (layer F.Cu) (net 17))
 (segment (start 125.87 102.97) (end 119 96.1) (width 0.254) (layer B.Cu) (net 17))
 (segment (start 127.02 112.54) (end 127.02 109.3) (width 0.254) (layer B.Cu) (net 17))
 (segment (start 127.02 109.3) (end 125.87 108.15) (width 0.254) (layer B.Cu) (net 17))
 (segment (start 125.87 108.15) (end 125.87 102.97) (width 0.254) (layer B.Cu) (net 17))
 (segment (start 122.98 80.72) (end 122.98 77.46) (width 0.254) (layer F.Cu) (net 17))
 (segment (start 124.13 81.87) (end 122.98 80.72) (width 0.254) (layer F.Cu) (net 17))
 (segment (start 124.13 90.97) (end 124.13 81.87) (width 0.254) (layer F.Cu) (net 17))
 (via (at 130.5 95.8) (size 0.889) (layers F.Cu B.Cu) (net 10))
 (via (at 130.5 102.3) (size 0.889) (layers F.Cu B.Cu) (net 12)) (via (at 119 100) (size 0.889) (layers F.Cu B.Cu) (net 20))
 (via (at 130.5 91.9) (size 0.889) (layers F.Cu B.Cu) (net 1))
 (via (at 130.5 93.2) (size 0.889) (layers F.Cu B.Cu) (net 11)) (via (at 119 97.4) (size 0.889) (layers F.Cu B.Cu) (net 18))
 (via (at 119 98.7) (size 0.889) (layers F.Cu B.Cu) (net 19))
 (via (at 131.9 93.3) (size 0.889) (layers F.Cu B.Cu) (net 22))
 (via (at 131.9 102.1) (size 0.889) (layers F.Cu B.Cu) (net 22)) (via (at 130.5 101) (size 0.889) (layers F.Cu B.Cu) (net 8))
 (via (at 130.5 99.7) (size 0.889) (layers F.Cu B.Cu) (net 13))
 (via (at 130.5 97.1) (size 0.889) (layers F.Cu B.Cu) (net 14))
 (via (at 130.5 94.5) (size 0.889) (layers F.Cu B.Cu) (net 15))
 (via (at 130.5 103.6) (size 0.889) (layers F.Cu B.Cu) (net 7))
 (via (at 130.5 98.4) (size 0.889) (layers F.Cu B.Cu) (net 9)) (via (at 119 94.8) (size 0.889) (layers F.Cu B.Cu) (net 16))
 (via (at 119 96.1) (size 0.889) (layers F.Cu B.Cu) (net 17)))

